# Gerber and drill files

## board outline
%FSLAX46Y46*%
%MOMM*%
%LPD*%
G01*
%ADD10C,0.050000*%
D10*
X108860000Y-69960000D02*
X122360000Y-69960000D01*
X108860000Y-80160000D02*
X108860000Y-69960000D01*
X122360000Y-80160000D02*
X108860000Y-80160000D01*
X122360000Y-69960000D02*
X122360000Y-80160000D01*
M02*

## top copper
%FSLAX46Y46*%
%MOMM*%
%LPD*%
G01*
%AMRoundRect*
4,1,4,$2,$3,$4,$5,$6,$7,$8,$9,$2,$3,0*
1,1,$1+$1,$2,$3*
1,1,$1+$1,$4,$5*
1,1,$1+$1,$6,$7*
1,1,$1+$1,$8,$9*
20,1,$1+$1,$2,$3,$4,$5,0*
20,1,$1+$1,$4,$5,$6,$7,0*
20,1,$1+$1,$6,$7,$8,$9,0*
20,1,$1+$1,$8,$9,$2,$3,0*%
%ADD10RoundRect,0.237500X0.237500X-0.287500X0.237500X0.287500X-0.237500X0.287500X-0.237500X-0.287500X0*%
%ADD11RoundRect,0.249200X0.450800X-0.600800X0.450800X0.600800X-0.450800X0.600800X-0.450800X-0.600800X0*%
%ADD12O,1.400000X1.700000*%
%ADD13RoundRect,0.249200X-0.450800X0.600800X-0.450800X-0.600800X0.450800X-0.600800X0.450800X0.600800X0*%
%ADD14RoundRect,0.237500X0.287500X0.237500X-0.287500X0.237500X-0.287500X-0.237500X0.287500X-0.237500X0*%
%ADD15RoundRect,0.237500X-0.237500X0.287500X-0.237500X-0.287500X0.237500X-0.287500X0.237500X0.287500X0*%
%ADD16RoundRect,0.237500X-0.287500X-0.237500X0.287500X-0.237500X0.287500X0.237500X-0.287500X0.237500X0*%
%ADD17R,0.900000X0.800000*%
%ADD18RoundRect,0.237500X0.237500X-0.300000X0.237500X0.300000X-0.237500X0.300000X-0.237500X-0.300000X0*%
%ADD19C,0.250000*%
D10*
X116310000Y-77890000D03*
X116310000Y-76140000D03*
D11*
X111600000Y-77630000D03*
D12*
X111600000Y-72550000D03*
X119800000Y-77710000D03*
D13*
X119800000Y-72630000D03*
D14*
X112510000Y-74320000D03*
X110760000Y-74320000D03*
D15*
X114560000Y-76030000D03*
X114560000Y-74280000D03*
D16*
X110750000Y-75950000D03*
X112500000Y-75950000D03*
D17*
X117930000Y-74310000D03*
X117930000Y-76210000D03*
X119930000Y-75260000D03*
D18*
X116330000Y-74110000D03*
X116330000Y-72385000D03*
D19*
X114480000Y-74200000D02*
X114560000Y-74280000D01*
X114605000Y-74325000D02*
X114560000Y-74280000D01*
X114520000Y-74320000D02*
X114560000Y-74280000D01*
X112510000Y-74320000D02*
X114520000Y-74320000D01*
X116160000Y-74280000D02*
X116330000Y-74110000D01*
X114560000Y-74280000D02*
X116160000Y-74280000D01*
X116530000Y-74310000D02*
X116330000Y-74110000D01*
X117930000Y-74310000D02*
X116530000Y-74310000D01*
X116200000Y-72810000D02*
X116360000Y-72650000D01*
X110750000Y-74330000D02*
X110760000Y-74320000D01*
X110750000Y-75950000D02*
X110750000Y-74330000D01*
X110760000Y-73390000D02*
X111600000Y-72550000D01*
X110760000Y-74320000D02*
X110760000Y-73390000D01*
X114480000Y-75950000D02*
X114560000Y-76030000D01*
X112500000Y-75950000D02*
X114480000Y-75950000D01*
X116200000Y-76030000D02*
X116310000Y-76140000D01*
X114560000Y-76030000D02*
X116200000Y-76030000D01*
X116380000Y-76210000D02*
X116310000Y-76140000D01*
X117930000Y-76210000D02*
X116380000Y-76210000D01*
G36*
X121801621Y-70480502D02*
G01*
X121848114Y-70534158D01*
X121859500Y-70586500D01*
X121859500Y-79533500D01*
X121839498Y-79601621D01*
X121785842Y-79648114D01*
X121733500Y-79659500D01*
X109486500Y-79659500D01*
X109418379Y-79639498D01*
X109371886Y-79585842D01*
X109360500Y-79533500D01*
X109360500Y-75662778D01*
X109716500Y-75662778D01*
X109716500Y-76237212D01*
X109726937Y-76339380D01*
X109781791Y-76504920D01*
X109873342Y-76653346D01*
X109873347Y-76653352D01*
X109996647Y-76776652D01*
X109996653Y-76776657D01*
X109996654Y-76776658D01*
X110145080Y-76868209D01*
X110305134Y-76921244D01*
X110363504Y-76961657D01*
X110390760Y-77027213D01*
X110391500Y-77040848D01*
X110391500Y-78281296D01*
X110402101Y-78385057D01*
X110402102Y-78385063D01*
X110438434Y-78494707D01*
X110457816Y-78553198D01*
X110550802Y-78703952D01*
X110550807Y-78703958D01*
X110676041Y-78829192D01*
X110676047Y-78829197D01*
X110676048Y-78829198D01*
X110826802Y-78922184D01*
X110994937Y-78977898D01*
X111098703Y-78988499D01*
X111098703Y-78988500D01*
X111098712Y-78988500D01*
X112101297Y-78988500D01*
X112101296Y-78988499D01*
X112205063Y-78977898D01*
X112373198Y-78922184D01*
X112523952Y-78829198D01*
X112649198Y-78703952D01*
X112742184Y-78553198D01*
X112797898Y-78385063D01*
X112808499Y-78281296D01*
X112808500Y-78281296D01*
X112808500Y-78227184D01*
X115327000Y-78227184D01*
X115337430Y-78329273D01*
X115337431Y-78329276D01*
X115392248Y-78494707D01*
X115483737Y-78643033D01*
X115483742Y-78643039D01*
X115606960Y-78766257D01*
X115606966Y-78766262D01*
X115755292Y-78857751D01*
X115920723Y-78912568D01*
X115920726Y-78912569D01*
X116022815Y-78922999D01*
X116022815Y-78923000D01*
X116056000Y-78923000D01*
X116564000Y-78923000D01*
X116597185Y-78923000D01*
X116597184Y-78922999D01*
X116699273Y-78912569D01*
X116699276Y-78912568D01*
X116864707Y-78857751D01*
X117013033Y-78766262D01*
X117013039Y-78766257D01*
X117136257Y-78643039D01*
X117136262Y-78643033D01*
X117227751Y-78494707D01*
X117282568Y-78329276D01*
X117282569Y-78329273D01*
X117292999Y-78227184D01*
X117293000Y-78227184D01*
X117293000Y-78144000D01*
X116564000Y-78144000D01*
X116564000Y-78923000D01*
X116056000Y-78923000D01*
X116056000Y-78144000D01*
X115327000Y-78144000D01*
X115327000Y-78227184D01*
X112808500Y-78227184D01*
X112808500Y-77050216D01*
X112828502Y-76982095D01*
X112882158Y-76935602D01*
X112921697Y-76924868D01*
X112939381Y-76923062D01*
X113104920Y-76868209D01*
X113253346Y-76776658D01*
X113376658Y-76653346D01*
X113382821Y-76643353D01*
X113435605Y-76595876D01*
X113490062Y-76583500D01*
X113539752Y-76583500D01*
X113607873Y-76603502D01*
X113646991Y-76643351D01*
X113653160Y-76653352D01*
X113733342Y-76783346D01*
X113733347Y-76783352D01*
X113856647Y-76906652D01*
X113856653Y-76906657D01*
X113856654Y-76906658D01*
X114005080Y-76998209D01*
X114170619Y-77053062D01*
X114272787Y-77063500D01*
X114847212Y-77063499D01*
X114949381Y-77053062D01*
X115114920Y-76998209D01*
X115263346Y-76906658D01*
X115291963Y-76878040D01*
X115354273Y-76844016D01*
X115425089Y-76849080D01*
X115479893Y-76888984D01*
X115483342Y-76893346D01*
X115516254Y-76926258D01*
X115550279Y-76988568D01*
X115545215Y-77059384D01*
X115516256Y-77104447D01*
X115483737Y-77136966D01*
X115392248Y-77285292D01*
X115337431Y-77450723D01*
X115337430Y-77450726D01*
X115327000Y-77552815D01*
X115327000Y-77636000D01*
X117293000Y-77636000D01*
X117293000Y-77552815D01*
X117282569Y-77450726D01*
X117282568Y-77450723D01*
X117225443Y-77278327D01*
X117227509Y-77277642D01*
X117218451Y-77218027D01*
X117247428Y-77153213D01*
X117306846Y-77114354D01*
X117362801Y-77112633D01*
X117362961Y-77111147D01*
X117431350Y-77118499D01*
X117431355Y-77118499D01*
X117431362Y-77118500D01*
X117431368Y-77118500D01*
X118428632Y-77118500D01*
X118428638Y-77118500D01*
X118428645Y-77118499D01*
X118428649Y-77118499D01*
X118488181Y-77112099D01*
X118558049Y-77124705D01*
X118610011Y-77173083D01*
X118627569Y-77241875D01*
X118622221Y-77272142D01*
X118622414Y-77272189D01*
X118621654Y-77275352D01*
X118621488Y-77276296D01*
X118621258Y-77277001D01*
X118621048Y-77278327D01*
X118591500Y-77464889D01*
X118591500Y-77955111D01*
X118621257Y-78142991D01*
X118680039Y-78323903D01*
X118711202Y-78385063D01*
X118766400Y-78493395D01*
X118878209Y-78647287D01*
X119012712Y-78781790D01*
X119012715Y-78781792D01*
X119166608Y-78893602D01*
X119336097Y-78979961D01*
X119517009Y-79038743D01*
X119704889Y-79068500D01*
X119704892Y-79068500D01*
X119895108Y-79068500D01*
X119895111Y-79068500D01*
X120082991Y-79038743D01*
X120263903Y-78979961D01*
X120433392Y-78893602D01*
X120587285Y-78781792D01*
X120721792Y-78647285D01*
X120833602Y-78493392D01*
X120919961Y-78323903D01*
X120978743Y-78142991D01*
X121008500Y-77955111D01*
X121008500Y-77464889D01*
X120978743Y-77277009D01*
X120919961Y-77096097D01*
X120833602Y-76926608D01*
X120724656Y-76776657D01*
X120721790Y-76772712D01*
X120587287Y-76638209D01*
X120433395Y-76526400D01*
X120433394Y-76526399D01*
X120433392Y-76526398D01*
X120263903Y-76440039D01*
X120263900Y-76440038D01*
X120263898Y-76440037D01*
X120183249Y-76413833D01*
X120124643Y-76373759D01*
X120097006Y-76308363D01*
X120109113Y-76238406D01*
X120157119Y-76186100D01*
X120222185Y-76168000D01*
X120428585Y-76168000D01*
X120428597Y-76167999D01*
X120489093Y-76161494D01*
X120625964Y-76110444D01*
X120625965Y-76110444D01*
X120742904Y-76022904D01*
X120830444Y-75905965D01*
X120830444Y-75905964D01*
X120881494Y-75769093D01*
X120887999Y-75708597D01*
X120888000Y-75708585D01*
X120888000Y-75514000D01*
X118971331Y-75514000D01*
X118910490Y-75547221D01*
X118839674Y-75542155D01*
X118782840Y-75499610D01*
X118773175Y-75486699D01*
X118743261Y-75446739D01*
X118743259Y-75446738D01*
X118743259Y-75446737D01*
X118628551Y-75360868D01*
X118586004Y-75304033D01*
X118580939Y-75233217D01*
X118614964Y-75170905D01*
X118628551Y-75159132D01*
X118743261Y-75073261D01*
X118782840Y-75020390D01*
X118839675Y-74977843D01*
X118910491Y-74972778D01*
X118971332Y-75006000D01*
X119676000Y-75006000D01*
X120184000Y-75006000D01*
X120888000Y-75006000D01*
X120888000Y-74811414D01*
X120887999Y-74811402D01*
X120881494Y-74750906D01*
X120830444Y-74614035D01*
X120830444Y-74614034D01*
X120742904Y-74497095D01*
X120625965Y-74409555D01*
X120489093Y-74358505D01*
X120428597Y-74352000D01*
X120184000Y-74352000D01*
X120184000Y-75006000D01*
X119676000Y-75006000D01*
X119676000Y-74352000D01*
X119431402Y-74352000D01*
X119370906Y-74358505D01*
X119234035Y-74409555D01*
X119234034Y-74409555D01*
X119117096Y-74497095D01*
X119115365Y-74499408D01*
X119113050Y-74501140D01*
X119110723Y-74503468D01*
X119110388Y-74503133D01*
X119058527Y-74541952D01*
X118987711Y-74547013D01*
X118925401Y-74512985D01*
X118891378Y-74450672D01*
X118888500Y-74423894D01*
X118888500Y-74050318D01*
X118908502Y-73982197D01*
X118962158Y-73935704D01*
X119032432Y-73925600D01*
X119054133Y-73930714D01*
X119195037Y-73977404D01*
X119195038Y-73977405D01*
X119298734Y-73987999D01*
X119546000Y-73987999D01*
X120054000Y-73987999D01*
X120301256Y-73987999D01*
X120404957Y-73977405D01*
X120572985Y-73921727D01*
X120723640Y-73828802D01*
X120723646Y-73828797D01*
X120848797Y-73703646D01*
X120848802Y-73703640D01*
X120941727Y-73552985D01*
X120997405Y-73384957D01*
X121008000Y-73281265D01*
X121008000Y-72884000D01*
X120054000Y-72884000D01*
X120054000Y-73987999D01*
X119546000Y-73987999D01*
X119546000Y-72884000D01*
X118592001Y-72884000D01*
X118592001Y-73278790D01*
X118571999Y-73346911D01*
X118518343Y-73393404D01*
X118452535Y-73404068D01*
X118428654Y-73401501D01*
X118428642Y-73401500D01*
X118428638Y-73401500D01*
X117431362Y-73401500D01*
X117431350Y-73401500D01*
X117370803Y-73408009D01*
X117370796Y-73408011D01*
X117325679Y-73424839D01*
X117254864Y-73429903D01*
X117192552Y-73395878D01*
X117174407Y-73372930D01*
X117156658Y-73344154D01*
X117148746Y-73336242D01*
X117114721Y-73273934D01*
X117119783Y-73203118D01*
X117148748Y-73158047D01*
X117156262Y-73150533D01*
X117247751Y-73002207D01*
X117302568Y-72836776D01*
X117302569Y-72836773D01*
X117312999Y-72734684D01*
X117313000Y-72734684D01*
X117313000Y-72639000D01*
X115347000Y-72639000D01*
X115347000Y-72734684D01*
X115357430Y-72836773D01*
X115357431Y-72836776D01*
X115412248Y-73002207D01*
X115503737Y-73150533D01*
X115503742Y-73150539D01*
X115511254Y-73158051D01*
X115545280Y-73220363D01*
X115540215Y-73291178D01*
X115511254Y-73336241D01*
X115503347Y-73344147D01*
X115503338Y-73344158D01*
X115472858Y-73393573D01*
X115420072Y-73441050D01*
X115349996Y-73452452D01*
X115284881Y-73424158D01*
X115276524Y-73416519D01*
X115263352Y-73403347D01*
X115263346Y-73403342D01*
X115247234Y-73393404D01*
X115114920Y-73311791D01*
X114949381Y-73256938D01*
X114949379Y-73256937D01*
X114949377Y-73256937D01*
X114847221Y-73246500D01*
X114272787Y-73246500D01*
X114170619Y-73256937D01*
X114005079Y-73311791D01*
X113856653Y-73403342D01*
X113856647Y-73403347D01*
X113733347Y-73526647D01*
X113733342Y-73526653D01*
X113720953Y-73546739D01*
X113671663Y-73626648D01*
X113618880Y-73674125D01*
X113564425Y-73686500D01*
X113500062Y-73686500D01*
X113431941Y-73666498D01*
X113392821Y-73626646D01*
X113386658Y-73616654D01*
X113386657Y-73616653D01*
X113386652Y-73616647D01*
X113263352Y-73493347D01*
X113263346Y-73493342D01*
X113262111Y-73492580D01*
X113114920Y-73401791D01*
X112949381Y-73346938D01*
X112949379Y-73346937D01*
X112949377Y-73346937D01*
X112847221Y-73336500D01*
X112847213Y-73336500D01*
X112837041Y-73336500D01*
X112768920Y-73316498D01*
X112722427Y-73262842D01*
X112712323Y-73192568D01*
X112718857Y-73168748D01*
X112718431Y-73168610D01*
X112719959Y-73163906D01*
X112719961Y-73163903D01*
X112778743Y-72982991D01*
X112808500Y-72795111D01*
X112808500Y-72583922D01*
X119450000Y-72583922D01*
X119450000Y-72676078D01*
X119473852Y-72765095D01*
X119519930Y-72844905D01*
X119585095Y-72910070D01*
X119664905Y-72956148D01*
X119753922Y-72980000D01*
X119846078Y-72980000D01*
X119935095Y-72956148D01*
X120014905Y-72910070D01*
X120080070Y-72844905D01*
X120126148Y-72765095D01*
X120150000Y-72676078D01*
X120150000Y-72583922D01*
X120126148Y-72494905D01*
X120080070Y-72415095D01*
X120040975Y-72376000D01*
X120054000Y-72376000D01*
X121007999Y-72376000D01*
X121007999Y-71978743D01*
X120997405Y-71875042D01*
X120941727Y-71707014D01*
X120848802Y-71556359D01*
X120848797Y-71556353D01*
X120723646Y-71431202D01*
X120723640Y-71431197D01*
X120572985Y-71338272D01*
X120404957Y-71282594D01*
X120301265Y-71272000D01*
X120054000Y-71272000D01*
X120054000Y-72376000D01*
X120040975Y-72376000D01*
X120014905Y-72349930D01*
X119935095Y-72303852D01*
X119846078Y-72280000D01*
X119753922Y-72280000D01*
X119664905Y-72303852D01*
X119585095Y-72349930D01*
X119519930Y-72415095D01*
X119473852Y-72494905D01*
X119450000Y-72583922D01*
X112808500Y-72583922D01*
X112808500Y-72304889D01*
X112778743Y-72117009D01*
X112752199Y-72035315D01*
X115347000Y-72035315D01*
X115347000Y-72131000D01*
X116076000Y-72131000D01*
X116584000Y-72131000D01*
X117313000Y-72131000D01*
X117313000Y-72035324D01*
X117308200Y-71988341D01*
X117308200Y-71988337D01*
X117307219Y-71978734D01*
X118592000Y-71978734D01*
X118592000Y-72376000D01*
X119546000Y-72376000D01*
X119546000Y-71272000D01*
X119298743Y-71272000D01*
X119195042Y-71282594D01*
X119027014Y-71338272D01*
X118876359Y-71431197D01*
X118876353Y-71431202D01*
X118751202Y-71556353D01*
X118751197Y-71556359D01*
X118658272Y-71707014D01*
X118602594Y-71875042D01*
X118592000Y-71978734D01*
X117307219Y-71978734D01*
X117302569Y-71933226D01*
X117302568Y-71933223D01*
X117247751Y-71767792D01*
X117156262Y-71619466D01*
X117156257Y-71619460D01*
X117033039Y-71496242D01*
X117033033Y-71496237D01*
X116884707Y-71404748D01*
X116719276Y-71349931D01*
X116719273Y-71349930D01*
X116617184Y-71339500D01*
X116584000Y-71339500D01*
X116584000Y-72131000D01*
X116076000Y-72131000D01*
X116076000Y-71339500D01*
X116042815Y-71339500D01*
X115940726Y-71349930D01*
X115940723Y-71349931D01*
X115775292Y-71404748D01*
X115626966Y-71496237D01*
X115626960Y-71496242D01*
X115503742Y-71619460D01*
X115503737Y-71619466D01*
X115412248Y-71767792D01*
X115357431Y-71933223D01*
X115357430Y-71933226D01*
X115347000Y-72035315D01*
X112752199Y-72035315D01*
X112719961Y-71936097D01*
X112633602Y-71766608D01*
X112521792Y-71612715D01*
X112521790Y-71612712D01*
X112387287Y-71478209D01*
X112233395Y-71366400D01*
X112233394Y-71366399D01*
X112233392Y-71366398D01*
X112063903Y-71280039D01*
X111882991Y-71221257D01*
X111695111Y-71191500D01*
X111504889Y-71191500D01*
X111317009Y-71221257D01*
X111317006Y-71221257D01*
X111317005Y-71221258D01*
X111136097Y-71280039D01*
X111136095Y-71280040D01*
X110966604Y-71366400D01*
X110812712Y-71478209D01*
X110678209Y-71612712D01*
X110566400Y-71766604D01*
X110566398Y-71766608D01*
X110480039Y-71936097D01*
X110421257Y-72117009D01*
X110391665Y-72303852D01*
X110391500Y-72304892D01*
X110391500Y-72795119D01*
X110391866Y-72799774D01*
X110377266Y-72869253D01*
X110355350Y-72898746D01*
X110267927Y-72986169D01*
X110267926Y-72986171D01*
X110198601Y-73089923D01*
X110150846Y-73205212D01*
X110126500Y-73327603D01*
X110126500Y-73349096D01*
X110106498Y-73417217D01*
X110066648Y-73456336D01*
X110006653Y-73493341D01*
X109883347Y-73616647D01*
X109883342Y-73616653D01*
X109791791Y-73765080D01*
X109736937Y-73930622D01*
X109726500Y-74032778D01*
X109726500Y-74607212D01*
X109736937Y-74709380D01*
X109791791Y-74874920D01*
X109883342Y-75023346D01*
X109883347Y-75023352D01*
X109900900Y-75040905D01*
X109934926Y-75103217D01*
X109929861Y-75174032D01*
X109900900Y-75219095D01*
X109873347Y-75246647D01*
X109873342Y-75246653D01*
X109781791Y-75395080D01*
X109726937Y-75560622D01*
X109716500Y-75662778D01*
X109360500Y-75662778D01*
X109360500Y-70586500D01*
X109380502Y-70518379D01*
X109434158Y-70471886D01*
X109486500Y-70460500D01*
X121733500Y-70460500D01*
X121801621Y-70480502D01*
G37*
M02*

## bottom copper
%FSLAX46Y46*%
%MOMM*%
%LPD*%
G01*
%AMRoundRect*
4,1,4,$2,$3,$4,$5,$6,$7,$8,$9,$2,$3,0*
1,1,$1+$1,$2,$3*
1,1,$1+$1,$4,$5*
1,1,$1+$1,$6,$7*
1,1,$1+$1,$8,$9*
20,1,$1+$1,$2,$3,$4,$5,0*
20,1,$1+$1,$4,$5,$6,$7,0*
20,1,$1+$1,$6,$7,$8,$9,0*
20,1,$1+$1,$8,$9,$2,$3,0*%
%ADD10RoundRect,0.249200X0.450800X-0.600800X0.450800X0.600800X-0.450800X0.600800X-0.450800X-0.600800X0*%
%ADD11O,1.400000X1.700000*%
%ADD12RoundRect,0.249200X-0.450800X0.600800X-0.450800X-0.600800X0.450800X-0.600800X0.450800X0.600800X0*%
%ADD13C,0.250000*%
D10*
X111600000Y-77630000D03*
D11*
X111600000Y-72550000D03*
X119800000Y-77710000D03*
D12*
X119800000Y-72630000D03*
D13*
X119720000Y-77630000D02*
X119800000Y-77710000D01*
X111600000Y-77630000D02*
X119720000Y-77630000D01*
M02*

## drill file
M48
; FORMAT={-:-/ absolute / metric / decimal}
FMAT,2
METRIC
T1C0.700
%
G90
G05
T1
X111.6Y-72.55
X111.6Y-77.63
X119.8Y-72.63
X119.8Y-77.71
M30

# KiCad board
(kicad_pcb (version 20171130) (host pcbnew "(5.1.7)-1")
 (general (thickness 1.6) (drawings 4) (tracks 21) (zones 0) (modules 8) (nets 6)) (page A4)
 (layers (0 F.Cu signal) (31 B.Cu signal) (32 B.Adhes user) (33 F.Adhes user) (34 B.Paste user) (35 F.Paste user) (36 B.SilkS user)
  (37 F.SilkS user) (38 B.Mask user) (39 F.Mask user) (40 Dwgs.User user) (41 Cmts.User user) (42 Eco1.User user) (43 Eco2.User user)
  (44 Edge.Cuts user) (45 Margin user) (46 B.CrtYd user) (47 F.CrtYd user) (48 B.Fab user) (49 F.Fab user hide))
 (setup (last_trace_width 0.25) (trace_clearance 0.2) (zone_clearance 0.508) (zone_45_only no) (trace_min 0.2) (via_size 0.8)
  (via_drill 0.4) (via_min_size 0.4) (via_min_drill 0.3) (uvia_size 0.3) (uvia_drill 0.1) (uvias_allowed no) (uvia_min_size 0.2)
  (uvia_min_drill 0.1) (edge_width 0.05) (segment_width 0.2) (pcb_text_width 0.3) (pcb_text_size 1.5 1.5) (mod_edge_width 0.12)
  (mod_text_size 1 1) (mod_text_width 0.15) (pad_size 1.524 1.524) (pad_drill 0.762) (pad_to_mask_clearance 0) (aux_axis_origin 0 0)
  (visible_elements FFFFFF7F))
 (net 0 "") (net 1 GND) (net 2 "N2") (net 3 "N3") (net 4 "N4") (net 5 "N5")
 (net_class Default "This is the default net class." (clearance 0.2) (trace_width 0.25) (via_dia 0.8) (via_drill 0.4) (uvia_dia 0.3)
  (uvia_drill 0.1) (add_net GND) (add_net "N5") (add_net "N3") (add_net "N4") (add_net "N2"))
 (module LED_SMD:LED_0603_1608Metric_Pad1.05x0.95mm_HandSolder (layer F.Cu) (at 116.31 77.015 90)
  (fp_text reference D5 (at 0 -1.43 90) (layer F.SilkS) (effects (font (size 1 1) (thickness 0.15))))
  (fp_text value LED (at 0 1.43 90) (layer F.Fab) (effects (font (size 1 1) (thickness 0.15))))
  (pad 1 smd roundrect (at -0.875 0 90) (size 1.05 0.95) (layers F.Cu F.Paste F.Mask) (roundrect_rratio 0.25) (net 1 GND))
  (pad 2 smd roundrect (at 0.875 0 90) (size 1.05 0.95) (layers F.Cu F.Paste F.Mask) (roundrect_rratio 0.25) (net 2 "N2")))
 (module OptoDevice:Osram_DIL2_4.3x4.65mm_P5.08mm (layer B.Cu) (at 111.6 77.63 90)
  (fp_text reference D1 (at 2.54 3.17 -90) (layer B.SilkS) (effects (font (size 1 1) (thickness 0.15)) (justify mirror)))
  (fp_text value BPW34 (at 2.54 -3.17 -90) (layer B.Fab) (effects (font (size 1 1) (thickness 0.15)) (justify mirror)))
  (pad 1 thru_hole roundrect (at 0 0 90) (size 1.7 1.4) (drill 0.7) (layers *.Cu *.Mask) (roundrect_rratio 0.178) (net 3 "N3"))
  (pad 2 thru_hole oval (at 5.08 0 90) (size 1.7 1.4) (drill 0.7) (layers *.Cu *.Mask) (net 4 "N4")))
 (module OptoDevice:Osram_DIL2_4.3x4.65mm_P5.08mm (layer B.Cu) (at 119.8 72.63 270)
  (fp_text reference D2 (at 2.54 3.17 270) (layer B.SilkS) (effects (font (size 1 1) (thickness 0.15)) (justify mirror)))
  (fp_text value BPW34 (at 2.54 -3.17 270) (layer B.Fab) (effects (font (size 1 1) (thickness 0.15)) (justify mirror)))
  (pad 2 thru_hole oval (at 5.08 0 270) (size 1.7 1.4) (drill 0.7) (layers *.Cu *.Mask) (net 3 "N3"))
  (pad 1 thru_hole roundrect (at 0 0 270) (size 1.7 1.4) (drill 0.7) (layers *.Cu *.Mask) (roundrect_rratio 0.178) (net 1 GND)))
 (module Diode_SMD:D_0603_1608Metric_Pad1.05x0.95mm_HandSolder (layer F.Cu) (at 111.635 74.32 180)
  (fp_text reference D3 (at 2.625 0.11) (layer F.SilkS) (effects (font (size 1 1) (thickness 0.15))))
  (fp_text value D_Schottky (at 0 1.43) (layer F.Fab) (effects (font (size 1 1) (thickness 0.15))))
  (pad 1 smd roundrect (at -0.875 0 180) (size 1.05 0.95) (layers F.Cu F.Paste F.Mask) (roundrect_rratio 0.25) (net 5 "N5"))
  (pad 2 smd roundrect (at 0.875 0 180) (size 1.05 0.95) (layers F.Cu F.Paste F.Mask) (roundrect_rratio 0.25) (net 4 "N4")))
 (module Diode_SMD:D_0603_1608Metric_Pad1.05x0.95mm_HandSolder (layer F.Cu) (at 114.56 75.155 270)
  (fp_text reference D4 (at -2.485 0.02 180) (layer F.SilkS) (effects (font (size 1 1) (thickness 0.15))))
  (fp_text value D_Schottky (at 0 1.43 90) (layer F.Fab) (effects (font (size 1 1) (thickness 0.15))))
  (pad 2 smd roundrect (at 0.875 0 270) (size 1.05 0.95) (layers F.Cu F.Paste F.Mask) (roundrect_rratio 0.25) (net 2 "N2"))
  (pad 1 smd roundrect (at -0.875 0 270) (size 1.05 0.95) (layers F.Cu F.Paste F.Mask) (roundrect_rratio 0.25) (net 5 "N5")))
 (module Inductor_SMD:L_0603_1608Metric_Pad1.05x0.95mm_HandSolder (layer F.Cu) (at 111.625 75.95)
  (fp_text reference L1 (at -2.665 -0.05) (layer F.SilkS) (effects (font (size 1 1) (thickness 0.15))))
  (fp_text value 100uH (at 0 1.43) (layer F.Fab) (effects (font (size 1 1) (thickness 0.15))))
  (pad 1 smd roundrect (at -0.875 0) (size 1.05 0.95) (layers F.Cu F.Paste F.Mask) (roundrect_rratio 0.25) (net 4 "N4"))
  (pad 2 smd roundrect (at 0.875 0) (size 1.05 0.95) (layers F.Cu F.Paste F.Mask) (roundrect_rratio 0.25) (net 2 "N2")))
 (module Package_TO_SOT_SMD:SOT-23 (layer F.Cu) (at 118.93 75.26)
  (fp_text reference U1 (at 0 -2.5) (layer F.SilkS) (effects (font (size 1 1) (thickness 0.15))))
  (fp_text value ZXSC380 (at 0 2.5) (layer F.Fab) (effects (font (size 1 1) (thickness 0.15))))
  (pad 1 smd rect (at -1 -0.95) (size 0.9 0.8) (layers F.Cu F.Paste F.Mask) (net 5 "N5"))
  (pad 2 smd rect (at -1 0.95) (size 0.9 0.8) (layers F.Cu F.Paste F.Mask) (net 2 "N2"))
  (pad 3 smd rect (at 1 0) (size 0.9 0.8) (layers F.Cu F.Paste F.Mask) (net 1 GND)))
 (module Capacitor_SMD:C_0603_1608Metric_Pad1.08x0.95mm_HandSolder (layer F.Cu) (at 116.33 73.2475 90)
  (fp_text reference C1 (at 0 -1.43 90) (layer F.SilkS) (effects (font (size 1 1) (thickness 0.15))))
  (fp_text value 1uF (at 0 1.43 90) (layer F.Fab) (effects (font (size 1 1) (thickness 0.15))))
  (pad 1 smd roundrect (at -0.8625 0 90) (size 1.075 0.95) (layers F.Cu F.Paste F.Mask) (roundrect_rratio 0.25) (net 5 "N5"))
  (pad 2 smd roundrect (at 0.8625 0 90) (size 1.075 0.95) (layers F.Cu F.Paste F.Mask) (roundrect_rratio 0.25) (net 1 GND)))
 (gr_line (start 108.86 69.96) (end 122.36 69.96) (layer Edge.Cuts) (width 0.05))
 (gr_line (start 108.86 80.16) (end 108.86 69.96) (layer Edge.Cuts) (width 0.05))
 (gr_line (start 122.36 80.16) (end 108.86 80.16) (layer Edge.Cuts) (width 0.05))
 (gr_line (start 122.36 69.96) (end 122.36 80.16) (layer Edge.Cuts) (width 0.05))
 (segment (start 114.48 74.2) (end 114.56 74.28) (width 0.25) (layer F.Cu) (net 5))
 (segment (start 114.605 74.325) (end 114.56 74.28) (width 0.25) (layer F.Cu) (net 5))
 (segment (start 114.52 74.32) (end 114.56 74.28) (width 0.25) (layer F.Cu) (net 5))
 (segment (start 112.51 74.32) (end 114.52 74.32) (width 0.25) (layer F.Cu) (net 5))
 (segment (start 116.16 74.28) (end 116.33 74.11) (width 0.25) (layer F.Cu) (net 5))
 (segment (start 114.56 74.28) (end 116.16 74.28) (width 0.25) (layer F.Cu) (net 5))
 (segment (start 116.53 74.31) (end 116.33 74.11) (width 0.25) (layer F.Cu) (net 5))
 (segment (start 117.93 74.31) (end 116.53 74.31) (width 0.25) (layer F.Cu) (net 5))
 (segment (start 119.72 77.63) (end 119.8 77.71) (width 0.25) (layer B.Cu) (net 3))
 (segment (start 111.6 77.63) (end 119.72 77.63) (width 0.25) (layer B.Cu) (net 3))
 (segment (start 116.2 72.81) (end 116.36 72.65) (width 0.25) (layer F.Cu) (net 1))
 (segment (start 110.75 74.33) (end 110.76 74.32) (width 0.25) (layer F.Cu) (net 4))
 (segment (start 110.75 75.95) (end 110.75 74.33) (width 0.25) (layer F.Cu) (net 4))
 (segment (start 110.76 73.39) (end 111.6 72.55) (width 0.25) (layer F.Cu) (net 4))
 (segment (start 110.76 74.32) (end 110.76 73.39) (width 0.25) (layer F.Cu) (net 4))
 (segment (start 114.48 75.95) (end 114.56 76.03) (width 0.25) (layer F.Cu) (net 2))
 (segment (start 112.5 75.95) (end 114.48 75.95) (width 0.25) (layer F.Cu) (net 2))
 (segment (start 116.2 76.03) (end 116.31 76.14) (width 0.25) (layer F.Cu) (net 2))
 (segment (start 114.56 76.03) (end 116.2 76.03) (width 0.25) (layer F.Cu) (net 2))
 (segment (start 116.38 76.21) (end 116.31 76.14) (width 0.25) (layer F.Cu) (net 2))
 (segment (start 117.93 76.21) (end 116.38 76.21) (width 0.25) (layer F.Cu) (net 2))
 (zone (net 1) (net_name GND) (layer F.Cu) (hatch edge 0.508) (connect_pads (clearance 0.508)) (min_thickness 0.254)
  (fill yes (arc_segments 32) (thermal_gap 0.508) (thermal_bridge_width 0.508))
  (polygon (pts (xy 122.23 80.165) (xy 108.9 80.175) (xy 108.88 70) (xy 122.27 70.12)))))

